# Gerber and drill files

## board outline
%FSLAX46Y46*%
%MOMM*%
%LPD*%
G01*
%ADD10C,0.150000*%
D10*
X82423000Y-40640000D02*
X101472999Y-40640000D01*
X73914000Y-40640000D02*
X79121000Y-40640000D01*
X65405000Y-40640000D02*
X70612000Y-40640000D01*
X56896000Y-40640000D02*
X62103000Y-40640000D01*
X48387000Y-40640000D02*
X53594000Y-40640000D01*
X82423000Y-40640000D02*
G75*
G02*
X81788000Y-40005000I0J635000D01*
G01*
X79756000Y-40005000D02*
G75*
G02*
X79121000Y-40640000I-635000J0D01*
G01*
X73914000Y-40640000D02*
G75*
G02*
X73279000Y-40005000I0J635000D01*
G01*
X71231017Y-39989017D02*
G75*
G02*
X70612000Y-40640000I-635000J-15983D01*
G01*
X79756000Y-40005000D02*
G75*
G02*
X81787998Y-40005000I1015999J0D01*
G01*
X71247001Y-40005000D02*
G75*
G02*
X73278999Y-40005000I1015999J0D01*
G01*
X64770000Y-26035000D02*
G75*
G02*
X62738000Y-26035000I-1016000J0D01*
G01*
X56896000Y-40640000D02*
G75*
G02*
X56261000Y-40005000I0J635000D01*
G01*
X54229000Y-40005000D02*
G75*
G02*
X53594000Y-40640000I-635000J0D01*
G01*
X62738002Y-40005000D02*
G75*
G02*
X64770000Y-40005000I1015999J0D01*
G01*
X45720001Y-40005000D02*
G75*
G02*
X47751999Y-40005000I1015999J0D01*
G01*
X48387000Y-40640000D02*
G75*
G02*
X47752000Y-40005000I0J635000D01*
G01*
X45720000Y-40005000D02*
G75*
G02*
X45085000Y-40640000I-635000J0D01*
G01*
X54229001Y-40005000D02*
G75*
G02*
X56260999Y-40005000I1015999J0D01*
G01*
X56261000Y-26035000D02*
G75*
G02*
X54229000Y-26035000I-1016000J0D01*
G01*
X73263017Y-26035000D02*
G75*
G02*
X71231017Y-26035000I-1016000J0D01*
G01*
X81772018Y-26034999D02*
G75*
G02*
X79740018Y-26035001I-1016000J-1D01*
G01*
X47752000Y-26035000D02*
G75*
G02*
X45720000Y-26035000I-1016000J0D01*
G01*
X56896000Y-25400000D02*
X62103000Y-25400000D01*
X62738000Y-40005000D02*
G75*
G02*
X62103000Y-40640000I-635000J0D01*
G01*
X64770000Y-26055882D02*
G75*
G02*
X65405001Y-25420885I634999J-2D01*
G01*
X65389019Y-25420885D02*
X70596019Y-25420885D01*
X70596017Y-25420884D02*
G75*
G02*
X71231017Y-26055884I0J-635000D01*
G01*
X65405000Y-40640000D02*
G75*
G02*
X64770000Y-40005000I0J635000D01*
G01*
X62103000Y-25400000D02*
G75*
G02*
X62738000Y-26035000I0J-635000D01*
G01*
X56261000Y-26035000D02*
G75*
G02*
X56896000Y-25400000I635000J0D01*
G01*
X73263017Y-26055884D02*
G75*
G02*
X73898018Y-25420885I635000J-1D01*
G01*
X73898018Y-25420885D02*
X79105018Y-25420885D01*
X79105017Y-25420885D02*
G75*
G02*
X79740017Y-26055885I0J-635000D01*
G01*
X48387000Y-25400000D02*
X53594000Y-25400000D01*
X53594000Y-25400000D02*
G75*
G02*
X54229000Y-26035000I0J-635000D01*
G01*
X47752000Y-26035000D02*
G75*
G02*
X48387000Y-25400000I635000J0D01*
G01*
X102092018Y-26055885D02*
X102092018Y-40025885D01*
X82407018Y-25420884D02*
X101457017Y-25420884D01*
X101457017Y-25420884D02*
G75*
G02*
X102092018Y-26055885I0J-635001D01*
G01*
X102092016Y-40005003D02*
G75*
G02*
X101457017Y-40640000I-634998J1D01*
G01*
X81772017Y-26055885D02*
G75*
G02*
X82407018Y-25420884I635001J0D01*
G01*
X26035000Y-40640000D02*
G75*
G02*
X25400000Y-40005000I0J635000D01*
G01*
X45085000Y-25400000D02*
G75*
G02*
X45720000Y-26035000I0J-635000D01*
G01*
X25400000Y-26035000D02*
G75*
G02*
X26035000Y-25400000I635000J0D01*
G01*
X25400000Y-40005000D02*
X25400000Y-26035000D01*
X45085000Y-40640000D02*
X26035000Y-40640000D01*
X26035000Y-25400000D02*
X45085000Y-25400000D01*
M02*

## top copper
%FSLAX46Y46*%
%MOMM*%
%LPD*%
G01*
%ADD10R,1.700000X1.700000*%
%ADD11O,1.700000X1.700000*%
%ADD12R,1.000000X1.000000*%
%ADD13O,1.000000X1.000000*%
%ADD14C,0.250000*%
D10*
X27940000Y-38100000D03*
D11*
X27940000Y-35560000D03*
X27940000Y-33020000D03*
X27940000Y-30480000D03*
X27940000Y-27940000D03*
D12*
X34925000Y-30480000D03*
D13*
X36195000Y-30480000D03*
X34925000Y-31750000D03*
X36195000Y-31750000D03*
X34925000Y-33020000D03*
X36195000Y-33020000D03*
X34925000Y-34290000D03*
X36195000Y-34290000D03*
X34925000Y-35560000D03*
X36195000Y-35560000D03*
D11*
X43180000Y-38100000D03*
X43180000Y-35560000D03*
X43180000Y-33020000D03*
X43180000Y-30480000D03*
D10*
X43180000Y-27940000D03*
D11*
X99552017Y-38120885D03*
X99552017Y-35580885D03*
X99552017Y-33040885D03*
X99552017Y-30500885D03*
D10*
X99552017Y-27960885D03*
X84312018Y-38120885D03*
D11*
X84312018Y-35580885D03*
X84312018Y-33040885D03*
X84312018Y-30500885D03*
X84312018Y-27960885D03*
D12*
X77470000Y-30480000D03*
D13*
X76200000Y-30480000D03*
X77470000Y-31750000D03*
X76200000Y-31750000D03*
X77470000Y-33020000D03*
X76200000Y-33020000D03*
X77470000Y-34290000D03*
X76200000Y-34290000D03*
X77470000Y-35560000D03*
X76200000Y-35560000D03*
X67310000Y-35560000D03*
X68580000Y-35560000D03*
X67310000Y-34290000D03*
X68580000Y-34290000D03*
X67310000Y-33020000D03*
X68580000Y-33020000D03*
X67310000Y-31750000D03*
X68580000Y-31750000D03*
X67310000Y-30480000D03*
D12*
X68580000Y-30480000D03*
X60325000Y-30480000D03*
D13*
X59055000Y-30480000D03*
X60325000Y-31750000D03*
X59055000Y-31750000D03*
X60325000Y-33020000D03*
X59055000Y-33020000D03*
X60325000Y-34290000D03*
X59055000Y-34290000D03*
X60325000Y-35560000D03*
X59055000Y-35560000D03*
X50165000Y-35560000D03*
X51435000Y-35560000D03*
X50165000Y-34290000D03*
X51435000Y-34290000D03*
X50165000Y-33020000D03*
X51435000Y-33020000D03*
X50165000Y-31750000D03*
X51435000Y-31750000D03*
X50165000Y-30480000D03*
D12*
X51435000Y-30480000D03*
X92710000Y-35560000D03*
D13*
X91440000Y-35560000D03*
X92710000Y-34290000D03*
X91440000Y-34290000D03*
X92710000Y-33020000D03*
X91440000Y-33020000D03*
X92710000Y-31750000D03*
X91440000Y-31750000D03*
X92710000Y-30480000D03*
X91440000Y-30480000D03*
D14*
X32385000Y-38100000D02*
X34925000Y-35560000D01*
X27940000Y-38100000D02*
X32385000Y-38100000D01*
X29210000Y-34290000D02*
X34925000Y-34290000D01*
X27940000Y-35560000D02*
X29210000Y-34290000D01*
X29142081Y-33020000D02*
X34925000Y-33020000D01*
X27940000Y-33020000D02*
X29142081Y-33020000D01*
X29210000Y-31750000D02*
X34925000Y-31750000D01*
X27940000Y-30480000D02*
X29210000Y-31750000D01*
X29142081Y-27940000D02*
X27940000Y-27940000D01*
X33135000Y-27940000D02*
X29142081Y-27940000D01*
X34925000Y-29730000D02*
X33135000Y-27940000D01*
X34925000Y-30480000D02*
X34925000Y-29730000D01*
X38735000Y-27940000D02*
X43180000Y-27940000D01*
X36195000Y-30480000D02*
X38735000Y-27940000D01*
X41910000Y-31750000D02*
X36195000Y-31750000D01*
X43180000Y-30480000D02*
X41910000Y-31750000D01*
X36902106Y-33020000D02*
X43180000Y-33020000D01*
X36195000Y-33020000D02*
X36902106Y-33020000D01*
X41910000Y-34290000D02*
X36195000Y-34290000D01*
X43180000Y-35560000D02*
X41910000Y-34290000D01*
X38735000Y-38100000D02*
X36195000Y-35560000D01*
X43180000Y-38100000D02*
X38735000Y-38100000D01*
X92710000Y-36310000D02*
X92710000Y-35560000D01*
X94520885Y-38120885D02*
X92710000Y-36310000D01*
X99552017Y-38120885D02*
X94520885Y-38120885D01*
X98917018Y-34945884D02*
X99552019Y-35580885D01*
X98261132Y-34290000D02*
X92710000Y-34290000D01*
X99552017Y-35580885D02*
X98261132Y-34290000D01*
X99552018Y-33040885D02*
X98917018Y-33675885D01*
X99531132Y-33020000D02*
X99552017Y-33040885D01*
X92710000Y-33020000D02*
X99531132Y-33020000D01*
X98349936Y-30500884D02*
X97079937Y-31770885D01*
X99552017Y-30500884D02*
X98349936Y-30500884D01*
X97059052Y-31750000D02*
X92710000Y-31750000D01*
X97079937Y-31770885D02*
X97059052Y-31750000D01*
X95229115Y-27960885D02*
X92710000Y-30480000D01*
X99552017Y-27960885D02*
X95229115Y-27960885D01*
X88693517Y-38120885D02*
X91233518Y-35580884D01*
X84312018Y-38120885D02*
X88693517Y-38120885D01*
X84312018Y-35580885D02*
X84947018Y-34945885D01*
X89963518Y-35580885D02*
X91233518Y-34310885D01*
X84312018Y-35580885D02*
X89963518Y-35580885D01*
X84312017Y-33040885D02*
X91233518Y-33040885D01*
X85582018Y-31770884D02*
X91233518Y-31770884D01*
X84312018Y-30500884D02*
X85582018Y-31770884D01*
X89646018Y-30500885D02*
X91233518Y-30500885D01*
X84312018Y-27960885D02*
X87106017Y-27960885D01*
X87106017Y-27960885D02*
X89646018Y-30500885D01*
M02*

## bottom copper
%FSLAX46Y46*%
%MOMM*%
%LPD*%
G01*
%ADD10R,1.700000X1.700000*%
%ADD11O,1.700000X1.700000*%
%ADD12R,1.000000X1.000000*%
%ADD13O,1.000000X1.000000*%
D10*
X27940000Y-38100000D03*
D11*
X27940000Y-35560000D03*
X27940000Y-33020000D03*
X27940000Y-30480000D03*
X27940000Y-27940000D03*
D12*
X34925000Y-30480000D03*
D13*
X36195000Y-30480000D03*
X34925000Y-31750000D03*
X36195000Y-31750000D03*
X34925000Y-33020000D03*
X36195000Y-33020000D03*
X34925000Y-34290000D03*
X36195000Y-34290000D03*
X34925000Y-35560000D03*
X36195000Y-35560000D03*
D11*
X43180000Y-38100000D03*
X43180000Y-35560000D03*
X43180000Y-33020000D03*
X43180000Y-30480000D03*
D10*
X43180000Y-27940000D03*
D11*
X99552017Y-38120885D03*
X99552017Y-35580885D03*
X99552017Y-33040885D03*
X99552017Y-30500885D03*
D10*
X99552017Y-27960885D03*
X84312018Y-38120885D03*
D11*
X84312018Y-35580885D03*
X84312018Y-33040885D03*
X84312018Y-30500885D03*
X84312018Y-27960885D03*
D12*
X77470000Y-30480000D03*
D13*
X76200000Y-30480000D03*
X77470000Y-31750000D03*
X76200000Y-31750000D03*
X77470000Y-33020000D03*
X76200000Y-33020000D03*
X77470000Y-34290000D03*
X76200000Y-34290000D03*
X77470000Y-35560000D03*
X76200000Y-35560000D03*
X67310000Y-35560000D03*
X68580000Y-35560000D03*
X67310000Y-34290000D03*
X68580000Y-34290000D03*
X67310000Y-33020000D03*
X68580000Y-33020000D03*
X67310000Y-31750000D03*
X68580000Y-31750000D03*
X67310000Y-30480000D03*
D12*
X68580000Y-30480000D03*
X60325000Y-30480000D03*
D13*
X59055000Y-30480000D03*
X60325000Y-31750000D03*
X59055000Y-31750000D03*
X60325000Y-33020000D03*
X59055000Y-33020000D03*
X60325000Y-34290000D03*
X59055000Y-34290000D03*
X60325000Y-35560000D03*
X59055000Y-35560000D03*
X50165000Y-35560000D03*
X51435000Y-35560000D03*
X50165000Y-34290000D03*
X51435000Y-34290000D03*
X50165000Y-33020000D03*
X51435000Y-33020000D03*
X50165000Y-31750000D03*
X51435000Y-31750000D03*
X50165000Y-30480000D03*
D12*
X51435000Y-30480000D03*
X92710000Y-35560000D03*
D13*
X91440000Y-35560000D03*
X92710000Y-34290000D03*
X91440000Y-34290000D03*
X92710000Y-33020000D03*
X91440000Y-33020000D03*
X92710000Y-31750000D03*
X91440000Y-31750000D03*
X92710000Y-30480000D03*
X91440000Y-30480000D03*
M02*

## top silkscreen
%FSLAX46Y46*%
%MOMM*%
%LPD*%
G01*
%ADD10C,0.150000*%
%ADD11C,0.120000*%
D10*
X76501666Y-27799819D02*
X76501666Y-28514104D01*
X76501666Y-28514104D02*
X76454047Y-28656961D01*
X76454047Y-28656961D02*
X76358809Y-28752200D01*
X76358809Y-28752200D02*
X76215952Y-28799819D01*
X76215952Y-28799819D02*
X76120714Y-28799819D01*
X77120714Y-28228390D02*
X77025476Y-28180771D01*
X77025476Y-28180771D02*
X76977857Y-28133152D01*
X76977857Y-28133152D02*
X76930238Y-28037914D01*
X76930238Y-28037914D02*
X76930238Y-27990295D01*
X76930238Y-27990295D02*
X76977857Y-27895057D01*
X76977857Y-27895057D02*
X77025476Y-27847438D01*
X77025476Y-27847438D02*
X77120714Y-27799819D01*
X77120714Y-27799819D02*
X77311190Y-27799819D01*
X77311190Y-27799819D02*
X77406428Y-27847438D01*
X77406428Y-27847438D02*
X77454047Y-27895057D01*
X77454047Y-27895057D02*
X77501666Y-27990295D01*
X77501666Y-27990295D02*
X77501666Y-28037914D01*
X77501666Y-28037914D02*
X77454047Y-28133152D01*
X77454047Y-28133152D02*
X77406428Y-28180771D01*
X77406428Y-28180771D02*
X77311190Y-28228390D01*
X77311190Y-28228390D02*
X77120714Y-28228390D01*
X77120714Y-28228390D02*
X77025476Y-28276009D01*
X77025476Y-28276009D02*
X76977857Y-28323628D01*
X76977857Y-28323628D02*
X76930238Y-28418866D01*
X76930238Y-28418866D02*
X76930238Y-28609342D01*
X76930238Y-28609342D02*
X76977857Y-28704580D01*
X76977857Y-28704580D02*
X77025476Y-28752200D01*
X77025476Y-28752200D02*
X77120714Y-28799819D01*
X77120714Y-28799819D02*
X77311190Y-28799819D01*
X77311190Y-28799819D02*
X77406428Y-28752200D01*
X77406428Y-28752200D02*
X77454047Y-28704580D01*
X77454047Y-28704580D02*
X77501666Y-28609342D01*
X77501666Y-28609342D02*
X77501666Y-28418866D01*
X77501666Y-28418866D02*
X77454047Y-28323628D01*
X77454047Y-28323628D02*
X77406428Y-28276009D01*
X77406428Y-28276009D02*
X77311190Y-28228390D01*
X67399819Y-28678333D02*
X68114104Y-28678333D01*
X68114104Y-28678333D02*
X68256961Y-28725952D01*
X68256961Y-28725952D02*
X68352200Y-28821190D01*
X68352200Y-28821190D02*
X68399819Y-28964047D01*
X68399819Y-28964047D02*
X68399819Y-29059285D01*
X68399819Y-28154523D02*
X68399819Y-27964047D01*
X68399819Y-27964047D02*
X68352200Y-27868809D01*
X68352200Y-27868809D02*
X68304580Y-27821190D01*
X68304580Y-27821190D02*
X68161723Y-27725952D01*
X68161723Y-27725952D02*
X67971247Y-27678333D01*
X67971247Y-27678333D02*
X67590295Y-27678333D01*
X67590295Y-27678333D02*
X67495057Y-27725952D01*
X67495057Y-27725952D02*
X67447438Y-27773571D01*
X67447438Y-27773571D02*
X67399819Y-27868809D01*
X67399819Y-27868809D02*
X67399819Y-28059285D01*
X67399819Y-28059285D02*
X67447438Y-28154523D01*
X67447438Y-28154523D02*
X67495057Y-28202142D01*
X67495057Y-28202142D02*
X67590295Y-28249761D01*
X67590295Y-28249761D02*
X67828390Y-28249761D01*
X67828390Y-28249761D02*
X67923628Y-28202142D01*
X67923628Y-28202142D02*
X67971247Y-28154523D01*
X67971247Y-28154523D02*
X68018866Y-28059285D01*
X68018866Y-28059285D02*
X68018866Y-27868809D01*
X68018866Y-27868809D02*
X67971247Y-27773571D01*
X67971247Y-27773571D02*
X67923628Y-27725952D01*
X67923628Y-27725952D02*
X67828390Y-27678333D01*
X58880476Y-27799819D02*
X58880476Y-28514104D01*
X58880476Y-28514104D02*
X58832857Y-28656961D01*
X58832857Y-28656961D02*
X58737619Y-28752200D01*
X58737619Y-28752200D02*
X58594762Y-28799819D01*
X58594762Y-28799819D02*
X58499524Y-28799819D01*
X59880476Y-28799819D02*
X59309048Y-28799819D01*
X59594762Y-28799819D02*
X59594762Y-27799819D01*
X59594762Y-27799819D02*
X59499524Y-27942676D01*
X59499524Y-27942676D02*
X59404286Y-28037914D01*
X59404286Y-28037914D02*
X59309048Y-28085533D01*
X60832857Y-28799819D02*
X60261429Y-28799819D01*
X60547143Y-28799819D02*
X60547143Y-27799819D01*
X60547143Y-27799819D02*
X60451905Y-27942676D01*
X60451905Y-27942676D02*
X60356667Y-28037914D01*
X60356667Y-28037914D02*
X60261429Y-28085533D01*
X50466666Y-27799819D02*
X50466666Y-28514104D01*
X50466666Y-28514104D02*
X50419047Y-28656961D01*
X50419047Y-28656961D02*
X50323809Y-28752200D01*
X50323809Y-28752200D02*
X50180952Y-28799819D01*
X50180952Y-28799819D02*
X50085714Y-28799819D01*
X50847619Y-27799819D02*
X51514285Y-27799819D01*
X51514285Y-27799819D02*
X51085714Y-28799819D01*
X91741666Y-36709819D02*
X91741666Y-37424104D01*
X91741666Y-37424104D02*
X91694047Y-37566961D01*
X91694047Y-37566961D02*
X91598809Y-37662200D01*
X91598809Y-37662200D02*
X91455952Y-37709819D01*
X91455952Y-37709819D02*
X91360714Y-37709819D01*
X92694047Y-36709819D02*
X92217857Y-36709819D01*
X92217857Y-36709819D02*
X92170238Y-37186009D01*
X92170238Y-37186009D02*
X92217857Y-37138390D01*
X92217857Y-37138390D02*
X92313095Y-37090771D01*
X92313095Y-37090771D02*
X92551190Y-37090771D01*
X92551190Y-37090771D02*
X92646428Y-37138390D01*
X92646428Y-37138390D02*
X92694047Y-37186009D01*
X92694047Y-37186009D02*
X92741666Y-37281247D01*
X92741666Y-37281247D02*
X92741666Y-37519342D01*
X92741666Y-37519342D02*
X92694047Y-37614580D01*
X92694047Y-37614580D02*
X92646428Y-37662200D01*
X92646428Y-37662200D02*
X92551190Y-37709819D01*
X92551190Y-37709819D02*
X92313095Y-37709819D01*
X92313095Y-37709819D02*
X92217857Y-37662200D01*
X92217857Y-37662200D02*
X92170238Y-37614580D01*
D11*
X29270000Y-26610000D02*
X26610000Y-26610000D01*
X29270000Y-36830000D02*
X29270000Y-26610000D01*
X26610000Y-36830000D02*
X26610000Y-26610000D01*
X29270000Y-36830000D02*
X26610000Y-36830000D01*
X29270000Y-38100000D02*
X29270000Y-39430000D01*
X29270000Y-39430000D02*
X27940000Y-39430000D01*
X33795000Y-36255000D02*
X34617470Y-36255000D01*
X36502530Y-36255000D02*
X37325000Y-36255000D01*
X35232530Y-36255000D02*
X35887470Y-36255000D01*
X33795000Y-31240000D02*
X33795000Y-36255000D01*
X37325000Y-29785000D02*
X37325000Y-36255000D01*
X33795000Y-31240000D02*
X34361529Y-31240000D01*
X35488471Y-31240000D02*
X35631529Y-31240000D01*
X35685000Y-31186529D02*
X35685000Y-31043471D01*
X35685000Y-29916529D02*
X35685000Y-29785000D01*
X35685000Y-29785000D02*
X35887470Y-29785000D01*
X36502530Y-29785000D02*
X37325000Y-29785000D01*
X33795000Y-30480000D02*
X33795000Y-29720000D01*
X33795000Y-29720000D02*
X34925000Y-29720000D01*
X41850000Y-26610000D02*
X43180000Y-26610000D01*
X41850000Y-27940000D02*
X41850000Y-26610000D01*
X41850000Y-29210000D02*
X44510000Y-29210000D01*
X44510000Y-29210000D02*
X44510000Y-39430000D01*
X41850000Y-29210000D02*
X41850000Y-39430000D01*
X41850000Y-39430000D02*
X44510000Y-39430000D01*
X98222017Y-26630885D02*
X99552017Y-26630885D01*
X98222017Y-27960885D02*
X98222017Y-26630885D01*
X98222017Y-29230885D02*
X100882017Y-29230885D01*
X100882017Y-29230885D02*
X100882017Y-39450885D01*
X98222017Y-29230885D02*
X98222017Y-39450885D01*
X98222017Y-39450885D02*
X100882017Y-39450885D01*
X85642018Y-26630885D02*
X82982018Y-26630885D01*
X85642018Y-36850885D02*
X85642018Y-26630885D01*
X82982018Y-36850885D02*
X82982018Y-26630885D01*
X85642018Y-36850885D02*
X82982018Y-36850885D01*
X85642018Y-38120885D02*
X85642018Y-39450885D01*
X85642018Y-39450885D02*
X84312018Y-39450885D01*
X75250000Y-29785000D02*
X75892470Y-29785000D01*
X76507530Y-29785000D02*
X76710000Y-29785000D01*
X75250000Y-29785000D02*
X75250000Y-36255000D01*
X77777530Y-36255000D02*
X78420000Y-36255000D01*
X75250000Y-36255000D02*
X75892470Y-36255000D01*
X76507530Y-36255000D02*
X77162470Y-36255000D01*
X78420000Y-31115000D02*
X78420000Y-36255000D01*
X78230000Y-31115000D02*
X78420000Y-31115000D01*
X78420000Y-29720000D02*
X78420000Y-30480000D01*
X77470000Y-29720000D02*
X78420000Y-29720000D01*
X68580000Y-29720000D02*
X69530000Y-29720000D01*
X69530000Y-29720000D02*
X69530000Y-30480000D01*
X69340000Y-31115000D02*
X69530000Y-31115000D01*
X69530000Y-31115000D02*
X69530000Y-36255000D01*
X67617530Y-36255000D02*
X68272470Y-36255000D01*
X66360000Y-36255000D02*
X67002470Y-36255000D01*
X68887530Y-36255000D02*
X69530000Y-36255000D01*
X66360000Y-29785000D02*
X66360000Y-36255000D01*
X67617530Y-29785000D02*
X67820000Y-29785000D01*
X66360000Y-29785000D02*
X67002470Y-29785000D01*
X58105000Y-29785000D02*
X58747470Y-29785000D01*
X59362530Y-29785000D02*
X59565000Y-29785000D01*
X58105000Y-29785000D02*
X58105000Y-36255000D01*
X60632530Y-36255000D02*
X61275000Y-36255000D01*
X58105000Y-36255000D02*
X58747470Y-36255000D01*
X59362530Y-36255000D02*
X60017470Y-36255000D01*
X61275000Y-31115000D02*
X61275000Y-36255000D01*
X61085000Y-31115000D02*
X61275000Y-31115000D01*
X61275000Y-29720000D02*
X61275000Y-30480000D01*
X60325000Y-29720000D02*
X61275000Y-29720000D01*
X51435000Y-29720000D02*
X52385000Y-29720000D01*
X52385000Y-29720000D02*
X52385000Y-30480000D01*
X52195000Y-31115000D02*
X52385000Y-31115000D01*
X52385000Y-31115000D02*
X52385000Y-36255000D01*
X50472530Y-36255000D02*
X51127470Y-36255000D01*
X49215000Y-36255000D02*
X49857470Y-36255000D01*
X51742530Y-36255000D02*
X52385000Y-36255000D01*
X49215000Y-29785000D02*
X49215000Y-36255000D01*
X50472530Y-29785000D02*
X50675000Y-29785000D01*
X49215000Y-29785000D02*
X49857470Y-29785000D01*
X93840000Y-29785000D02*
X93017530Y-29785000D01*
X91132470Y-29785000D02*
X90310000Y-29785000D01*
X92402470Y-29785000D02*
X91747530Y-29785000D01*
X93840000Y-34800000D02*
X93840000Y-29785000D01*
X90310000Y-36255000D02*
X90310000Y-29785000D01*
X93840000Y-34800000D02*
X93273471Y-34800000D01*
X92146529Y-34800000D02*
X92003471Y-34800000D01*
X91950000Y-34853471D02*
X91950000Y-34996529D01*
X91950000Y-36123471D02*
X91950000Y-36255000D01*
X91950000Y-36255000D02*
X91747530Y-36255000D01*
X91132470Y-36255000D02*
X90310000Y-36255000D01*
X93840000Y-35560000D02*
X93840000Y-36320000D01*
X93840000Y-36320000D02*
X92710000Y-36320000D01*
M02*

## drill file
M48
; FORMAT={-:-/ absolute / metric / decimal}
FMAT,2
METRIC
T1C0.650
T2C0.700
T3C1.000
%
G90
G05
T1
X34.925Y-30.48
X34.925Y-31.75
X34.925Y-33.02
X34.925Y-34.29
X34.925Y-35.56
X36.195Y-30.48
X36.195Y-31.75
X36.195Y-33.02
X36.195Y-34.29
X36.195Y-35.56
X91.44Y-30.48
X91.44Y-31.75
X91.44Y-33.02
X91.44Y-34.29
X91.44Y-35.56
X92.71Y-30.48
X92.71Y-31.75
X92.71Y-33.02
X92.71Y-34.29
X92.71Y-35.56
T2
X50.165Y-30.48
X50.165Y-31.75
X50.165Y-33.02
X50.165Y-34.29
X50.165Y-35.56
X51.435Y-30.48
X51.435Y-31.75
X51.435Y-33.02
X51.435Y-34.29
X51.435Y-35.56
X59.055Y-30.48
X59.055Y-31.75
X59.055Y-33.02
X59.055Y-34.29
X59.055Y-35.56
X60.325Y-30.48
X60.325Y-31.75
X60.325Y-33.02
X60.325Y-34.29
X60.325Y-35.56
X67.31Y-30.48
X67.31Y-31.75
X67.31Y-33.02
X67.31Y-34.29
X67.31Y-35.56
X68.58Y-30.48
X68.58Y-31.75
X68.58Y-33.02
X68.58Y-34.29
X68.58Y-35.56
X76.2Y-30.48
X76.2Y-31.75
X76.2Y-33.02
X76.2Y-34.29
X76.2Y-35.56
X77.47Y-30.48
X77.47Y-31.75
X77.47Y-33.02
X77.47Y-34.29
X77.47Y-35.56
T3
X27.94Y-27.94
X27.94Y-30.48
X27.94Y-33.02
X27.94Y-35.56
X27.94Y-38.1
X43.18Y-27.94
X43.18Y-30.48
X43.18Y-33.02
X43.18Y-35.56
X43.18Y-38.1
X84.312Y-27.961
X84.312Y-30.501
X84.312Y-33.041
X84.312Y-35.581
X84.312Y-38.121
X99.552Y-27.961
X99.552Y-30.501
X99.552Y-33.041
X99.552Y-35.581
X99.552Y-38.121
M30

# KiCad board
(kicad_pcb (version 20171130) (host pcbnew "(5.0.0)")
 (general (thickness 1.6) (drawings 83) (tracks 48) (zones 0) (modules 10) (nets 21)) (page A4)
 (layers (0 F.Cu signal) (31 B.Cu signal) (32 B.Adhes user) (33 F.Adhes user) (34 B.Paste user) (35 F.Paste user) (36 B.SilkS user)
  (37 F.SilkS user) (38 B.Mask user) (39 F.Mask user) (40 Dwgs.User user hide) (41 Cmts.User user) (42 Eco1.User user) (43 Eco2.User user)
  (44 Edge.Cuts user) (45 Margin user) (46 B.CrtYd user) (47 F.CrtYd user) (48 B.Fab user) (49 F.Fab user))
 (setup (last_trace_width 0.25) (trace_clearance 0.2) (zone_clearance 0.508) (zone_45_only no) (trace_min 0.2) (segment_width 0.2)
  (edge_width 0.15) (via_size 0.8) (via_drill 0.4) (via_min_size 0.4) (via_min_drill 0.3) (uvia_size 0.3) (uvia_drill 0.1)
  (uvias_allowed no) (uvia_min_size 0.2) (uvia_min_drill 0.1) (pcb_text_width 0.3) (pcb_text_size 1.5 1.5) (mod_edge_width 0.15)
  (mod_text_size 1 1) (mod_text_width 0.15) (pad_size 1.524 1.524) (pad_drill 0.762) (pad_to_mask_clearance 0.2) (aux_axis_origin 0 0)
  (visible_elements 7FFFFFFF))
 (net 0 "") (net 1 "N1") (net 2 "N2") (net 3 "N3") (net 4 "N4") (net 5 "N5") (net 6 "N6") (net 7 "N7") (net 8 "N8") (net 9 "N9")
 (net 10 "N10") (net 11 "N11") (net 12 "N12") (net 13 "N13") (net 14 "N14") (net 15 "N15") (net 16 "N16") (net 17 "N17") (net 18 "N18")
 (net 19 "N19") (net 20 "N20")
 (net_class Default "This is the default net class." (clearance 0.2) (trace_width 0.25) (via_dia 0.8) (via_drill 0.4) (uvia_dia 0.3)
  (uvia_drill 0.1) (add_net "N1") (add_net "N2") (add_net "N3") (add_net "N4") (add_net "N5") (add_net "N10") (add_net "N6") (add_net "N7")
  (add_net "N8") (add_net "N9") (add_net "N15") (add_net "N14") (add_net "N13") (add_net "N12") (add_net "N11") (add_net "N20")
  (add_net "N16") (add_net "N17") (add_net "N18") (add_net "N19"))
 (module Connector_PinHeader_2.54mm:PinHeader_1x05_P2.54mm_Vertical (layer F.Cu) (at 27.94 38.1 180)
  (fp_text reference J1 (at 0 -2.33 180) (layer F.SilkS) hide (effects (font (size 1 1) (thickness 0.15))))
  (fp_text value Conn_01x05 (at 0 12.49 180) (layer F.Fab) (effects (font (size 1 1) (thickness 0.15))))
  (fp_line (start -1.33 11.49) (end 1.33 11.49) (layer F.SilkS) (width 0.12))
  (fp_line (start -1.33 1.27) (end -1.33 11.49) (layer F.SilkS) (width 0.12))
  (fp_line (start 1.33 1.27) (end 1.33 11.49) (layer F.SilkS) (width 0.12))
  (fp_line (start -1.33 1.27) (end 1.33 1.27) (layer F.SilkS) (width 0.12))
  (fp_line (start -1.33 0) (end -1.33 -1.33) (layer F.SilkS) (width 0.12))
  (fp_line (start -1.33 -1.33) (end 0 -1.33) (layer F.SilkS) (width 0.12))
  (pad 1 thru_hole rect (at 0 0 180) (size 1.7 1.7) (drill 1) (layers *.Cu *.Mask) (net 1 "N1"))
  (pad 2 thru_hole oval (at 0 2.54 180) (size 1.7 1.7) (drill 1) (layers *.Cu *.Mask) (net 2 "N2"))
  (pad 3 thru_hole oval (at 0 5.08 180) (size 1.7 1.7) (drill 1) (layers *.Cu *.Mask) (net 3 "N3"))
  (pad 4 thru_hole oval (at 0 7.62 180) (size 1.7 1.7) (drill 1) (layers *.Cu *.Mask) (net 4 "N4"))
  (pad 5 thru_hole oval (at 0 10.16 180) (size 1.7 1.7) (drill 1) (layers *.Cu *.Mask) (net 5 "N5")))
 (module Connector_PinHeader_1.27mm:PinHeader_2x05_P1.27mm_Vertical (layer F.Cu) (at 34.925 30.48)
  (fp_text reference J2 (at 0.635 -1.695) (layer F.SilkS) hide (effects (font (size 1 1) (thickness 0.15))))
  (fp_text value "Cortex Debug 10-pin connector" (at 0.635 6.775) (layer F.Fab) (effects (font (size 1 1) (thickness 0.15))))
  (fp_line (start -1.13 5.775) (end -0.30753 5.775) (layer F.SilkS) (width 0.12))
  (fp_line (start 1.57753 5.775) (end 2.4 5.775) (layer F.SilkS) (width 0.12))
  (fp_line (start 0.30753 5.775) (end 0.96247 5.775) (layer F.SilkS) (width 0.12))
  (fp_line (start -1.13 0.76) (end -1.13 5.775) (layer F.SilkS) (width 0.12))
  (fp_line (start 2.4 -0.695) (end 2.4 5.775) (layer F.SilkS) (width 0.12))
  (fp_line (start -1.13 0.76) (end -0.563471 0.76) (layer F.SilkS) (width 0.12))
  (fp_line (start 0.563471 0.76) (end 0.706529 0.76) (layer F.SilkS) (width 0.12))
  (fp_line (start 0.76 0.706529) (end 0.76 0.563471) (layer F.SilkS) (width 0.12))
  (fp_line (start 0.76 -0.563471) (end 0.76 -0.695) (layer F.SilkS) (width 0.12))
  (fp_line (start 0.76 -0.695) (end 0.96247 -0.695) (layer F.SilkS) (width 0.12))
  (fp_line (start 1.57753 -0.695) (end 2.4 -0.695) (layer F.SilkS) (width 0.12))
  (fp_line (start -1.13 0) (end -1.13 -0.76) (layer F.SilkS) (width 0.12))
  (fp_line (start -1.13 -0.76) (end 0 -0.76) (layer F.SilkS) (width 0.12))
  (pad 1 thru_hole rect (at 0 0) (size 1 1) (drill 0.65) (layers *.Cu *.Mask) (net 5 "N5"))
  (pad 2 thru_hole oval (at 1.27 0) (size 1 1) (drill 0.65) (layers *.Cu *.Mask) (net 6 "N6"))
  (pad 3 thru_hole oval (at 0 1.27) (size 1 1) (drill 0.65) (layers *.Cu *.Mask) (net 4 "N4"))
  (pad 4 thru_hole oval (at 1.27 1.27) (size 1 1) (drill 0.65) (layers *.Cu *.Mask) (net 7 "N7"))
  (pad 5 thru_hole oval (at 0 2.54) (size 1 1) (drill 0.65) (layers *.Cu *.Mask) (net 3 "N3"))
  (pad 6 thru_hole oval (at 1.27 2.54) (size 1 1) (drill 0.65) (layers *.Cu *.Mask) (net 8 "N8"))
  (pad 7 thru_hole oval (at 0 3.81) (size 1 1) (drill 0.65) (layers *.Cu *.Mask) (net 2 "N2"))
  (pad 8 thru_hole oval (at 1.27 3.81) (size 1 1) (drill 0.65) (layers *.Cu *.Mask) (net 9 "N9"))
  (pad 9 thru_hole oval (at 0 5.08) (size 1 1) (drill 0.65) (layers *.Cu *.Mask) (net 1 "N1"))
  (pad 10 thru_hole oval (at 1.27 5.08) (size 1 1) (drill 0.65) (layers *.Cu *.Mask) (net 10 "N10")))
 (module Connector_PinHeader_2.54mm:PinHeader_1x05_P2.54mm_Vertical (layer F.Cu) (at 43.18 27.94)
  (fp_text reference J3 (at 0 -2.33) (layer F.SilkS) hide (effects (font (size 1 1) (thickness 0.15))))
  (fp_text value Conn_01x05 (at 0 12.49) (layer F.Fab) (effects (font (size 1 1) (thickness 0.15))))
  (fp_line (start -1.33 -1.33) (end 0 -1.33) (layer F.SilkS) (width 0.12))
  (fp_line (start -1.33 0) (end -1.33 -1.33) (layer F.SilkS) (width 0.12))
  (fp_line (start -1.33 1.27) (end 1.33 1.27) (layer F.SilkS) (width 0.12))
  (fp_line (start 1.33 1.27) (end 1.33 11.49) (layer F.SilkS) (width 0.12))
  (fp_line (start -1.33 1.27) (end -1.33 11.49) (layer F.SilkS) (width 0.12))
  (fp_line (start -1.33 11.49) (end 1.33 11.49) (layer F.SilkS) (width 0.12))
  (pad 5 thru_hole oval (at 0 10.16) (size 1.7 1.7) (drill 1) (layers *.Cu *.Mask) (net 10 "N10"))
  (pad 4 thru_hole oval (at 0 7.62) (size 1.7 1.7) (drill 1) (layers *.Cu *.Mask) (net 9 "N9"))
  (pad 3 thru_hole oval (at 0 5.08) (size 1.7 1.7) (drill 1) (layers *.Cu *.Mask) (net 8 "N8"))
  (pad 2 thru_hole oval (at 0 2.54) (size 1.7 1.7) (drill 1) (layers *.Cu *.Mask) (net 7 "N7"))
  (pad 1 thru_hole rect (at 0 0) (size 1.7 1.7) (drill 1) (layers *.Cu *.Mask) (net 6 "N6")))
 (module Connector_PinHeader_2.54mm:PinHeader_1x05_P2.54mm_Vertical (layer F.Cu) (at 99.552017 27.960885)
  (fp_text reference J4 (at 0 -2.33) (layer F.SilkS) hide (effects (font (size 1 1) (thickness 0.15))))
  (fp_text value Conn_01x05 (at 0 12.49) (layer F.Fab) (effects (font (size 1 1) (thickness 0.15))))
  (fp_line (start -1.33 -1.33) (end 0 -1.33) (layer F.SilkS) (width 0.12))
  (fp_line (start -1.33 0) (end -1.33 -1.33) (layer F.SilkS) (width 0.12))
  (fp_line (start -1.33 1.27) (end 1.33 1.27) (layer F.SilkS) (width 0.12))
  (fp_line (start 1.33 1.27) (end 1.33 11.49) (layer F.SilkS) (width 0.12))
  (fp_line (start -1.33 1.27) (end -1.33 11.49) (layer F.SilkS) (width 0.12))
  (fp_line (start -1.33 11.49) (end 1.33 11.49) (layer F.SilkS) (width 0.12))
  (pad 5 thru_hole oval (at 0 10.16) (size 1.7 1.7) (drill 1) (layers *.Cu *.Mask) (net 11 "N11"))
  (pad 4 thru_hole oval (at 0 7.62) (size 1.7 1.7) (drill 1) (layers *.Cu *.Mask) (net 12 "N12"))
  (pad 3 thru_hole oval (at 0 5.08) (size 1.7 1.7) (drill 1) (layers *.Cu *.Mask) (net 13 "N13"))
  (pad 2 thru_hole oval (at 0 2.54) (size 1.7 1.7) (drill 1) (layers *.Cu *.Mask) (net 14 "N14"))
  (pad 1 thru_hole rect (at 0 0) (size 1.7 1.7) (drill 1) (layers *.Cu *.Mask) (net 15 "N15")))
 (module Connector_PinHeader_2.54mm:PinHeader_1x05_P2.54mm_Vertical (layer F.Cu) (at 84.312018 38.120885 180)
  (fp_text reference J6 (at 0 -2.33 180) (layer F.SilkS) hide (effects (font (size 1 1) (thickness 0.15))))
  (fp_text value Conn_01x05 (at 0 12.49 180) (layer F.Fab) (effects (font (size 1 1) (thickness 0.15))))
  (fp_line (start -1.33 11.49) (end 1.33 11.49) (layer F.SilkS) (width 0.12))
  (fp_line (start -1.33 1.27) (end -1.33 11.49) (layer F.SilkS) (width 0.12))
  (fp_line (start 1.33 1.27) (end 1.33 11.49) (layer F.SilkS) (width 0.12))
  (fp_line (start -1.33 1.27) (end 1.33 1.27) (layer F.SilkS) (width 0.12))
  (fp_line (start -1.33 0) (end -1.33 -1.33) (layer F.SilkS) (width 0.12))
  (fp_line (start -1.33 -1.33) (end 0 -1.33) (layer F.SilkS) (width 0.12))
  (pad 1 thru_hole rect (at 0 0 180) (size 1.7 1.7) (drill 1) (layers *.Cu *.Mask) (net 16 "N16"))
  (pad 2 thru_hole oval (at 0 2.54 180) (size 1.7 1.7) (drill 1) (layers *.Cu *.Mask) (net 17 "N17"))
  (pad 3 thru_hole oval (at 0 5.08 180) (size 1.7 1.7) (drill 1) (layers *.Cu *.Mask) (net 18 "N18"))
  (pad 4 thru_hole oval (at 0 7.62 180) (size 1.7 1.7) (drill 1) (layers *.Cu *.Mask) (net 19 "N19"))
  (pad 5 thru_hole oval (at 0 10.16 180) (size 1.7 1.7) (drill 1) (layers *.Cu *.Mask) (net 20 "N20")))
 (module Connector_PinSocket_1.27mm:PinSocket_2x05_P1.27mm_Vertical (layer F.Cu) (at 77.47 30.48)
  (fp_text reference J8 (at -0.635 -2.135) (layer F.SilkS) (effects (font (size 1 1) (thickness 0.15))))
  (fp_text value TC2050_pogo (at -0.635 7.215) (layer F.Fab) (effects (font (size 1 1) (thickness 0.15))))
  (fp_line (start -2.22 -0.695) (end -1.57753 -0.695) (layer F.SilkS) (width 0.12))
  (fp_line (start -0.96247 -0.695) (end -0.76 -0.695) (layer F.SilkS) (width 0.12))
  (fp_line (start -2.22 -0.695) (end -2.22 5.775) (layer F.SilkS) (width 0.12))
  (fp_line (start 0.30753 5.775) (end 0.95 5.775) (layer F.SilkS) (width 0.12))
  (fp_line (start -2.22 5.775) (end -1.57753 5.775) (layer F.SilkS) (width 0.12))
  (fp_line (start -0.96247 5.775) (end -0.30753 5.775) (layer F.SilkS) (width 0.12))
  (fp_line (start 0.95 0.635) (end 0.95 5.775) (layer F.SilkS) (width 0.12))
  (fp_line (start 0.76 0.635) (end 0.95 0.635) (layer F.SilkS) (width 0.12))
  (fp_line (start 0.95 -0.76) (end 0.95 0) (layer F.SilkS) (width 0.12))
  (fp_line (start 0 -0.76) (end 0.95 -0.76) (layer F.SilkS) (width 0.12))
  (pad 1 thru_hole rect (at 0 0) (size 1 1) (drill 0.7) (layers *.Cu *.Mask))
  (pad 2 thru_hole oval (at -1.27 0) (size 1 1) (drill 0.7) (layers *.Cu *.Mask))
  (pad 3 thru_hole oval (at 0 1.27) (size 1 1) (drill 0.7) (layers *.Cu *.Mask))
  (pad 4 thru_hole oval (at -1.27 1.27) (size 1 1) (drill 0.7) (layers *.Cu *.Mask))
  (pad 5 thru_hole oval (at 0 2.54) (size 1 1) (drill 0.7) (layers *.Cu *.Mask))
  (pad 6 thru_hole oval (at -1.27 2.54) (size 1 1) (drill 0.7) (layers *.Cu *.Mask))
  (pad 7 thru_hole oval (at 0 3.81) (size 1 1) (drill 0.7) (layers *.Cu *.Mask))
  (pad 8 thru_hole oval (at -1.27 3.81) (size 1 1) (drill 0.7) (layers *.Cu *.Mask))
  (pad 9 thru_hole oval (at 0 5.08) (size 1 1) (drill 0.7) (layers *.Cu *.Mask))
  (pad 10 thru_hole oval (at -1.27 5.08) (size 1 1) (drill 0.7) (layers *.Cu *.Mask)))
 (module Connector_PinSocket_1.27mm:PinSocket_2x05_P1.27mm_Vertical (layer F.Cu) (at 68.58 30.48)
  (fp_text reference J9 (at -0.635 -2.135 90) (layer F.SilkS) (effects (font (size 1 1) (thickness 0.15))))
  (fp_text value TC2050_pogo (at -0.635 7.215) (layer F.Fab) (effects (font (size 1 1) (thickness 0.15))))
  (fp_line (start 0 -0.76) (end 0.95 -0.76) (layer F.SilkS) (width 0.12))
  (fp_line (start 0.95 -0.76) (end 0.95 0) (layer F.SilkS) (width 0.12))
  (fp_line (start 0.76 0.635) (end 0.95 0.635) (layer F.SilkS) (width 0.12))
  (fp_line (start 0.95 0.635) (end 0.95 5.775) (layer F.SilkS) (width 0.12))
  (fp_line (start -0.96247 5.775) (end -0.30753 5.775) (layer F.SilkS) (width 0.12))
  (fp_line (start -2.22 5.775) (end -1.57753 5.775) (layer F.SilkS) (width 0.12))
  (fp_line (start 0.30753 5.775) (end 0.95 5.775) (layer F.SilkS) (width 0.12))
  (fp_line (start -2.22 -0.695) (end -2.22 5.775) (layer F.SilkS) (width 0.12))
  (fp_line (start -0.96247 -0.695) (end -0.76 -0.695) (layer F.SilkS) (width 0.12))
  (fp_line (start -2.22 -0.695) (end -1.57753 -0.695) (layer F.SilkS) (width 0.12))
  (pad 10 thru_hole oval (at -1.27 5.08) (size 1 1) (drill 0.7) (layers *.Cu *.Mask))
  (pad 9 thru_hole oval (at 0 5.08) (size 1 1) (drill 0.7) (layers *.Cu *.Mask))
  (pad 8 thru_hole oval (at -1.27 3.81) (size 1 1) (drill 0.7) (layers *.Cu *.Mask))
  (pad 7 thru_hole oval (at 0 3.81) (size 1 1) (drill 0.7) (layers *.Cu *.Mask))
  (pad 6 thru_hole oval (at -1.27 2.54) (size 1 1) (drill 0.7) (layers *.Cu *.Mask))
  (pad 5 thru_hole oval (at 0 2.54) (size 1 1) (drill 0.7) (layers *.Cu *.Mask))
  (pad 4 thru_hole oval (at -1.27 1.27) (size 1 1) (drill 0.7) (layers *.Cu *.Mask))
  (pad 3 thru_hole oval (at 0 1.27) (size 1 1) (drill 0.7) (layers *.Cu *.Mask))
  (pad 2 thru_hole oval (at -1.27 0) (size 1 1) (drill 0.7) (layers *.Cu *.Mask))
  (pad 1 thru_hole rect (at 0 0) (size 1 1) (drill 0.7) (layers *.Cu *.Mask)))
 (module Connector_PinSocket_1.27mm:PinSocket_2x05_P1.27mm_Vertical (layer F.Cu) (at 60.325 30.48)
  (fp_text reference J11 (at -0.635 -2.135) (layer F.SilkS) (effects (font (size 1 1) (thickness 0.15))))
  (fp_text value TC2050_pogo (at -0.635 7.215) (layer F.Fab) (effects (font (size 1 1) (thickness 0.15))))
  (fp_line (start -2.22 -0.695) (end -1.57753 -0.695) (layer F.SilkS) (width 0.12))
  (fp_line (start -0.96247 -0.695) (end -0.76 -0.695) (layer F.SilkS) (width 0.12))
  (fp_line (start -2.22 -0.695) (end -2.22 5.775) (layer F.SilkS) (width 0.12))
  (fp_line (start 0.30753 5.775) (end 0.95 5.775) (layer F.SilkS) (width 0.12))
  (fp_line (start -2.22 5.775) (end -1.57753 5.775) (layer F.SilkS) (width 0.12))
  (fp_line (start -0.96247 5.775) (end -0.30753 5.775) (layer F.SilkS) (width 0.12))
  (fp_line (start 0.95 0.635) (end 0.95 5.775) (layer F.SilkS) (width 0.12))
  (fp_line (start 0.76 0.635) (end 0.95 0.635) (layer F.SilkS) (width 0.12))
  (fp_line (start 0.95 -0.76) (end 0.95 0) (layer F.SilkS) (width 0.12))
  (fp_line (start 0 -0.76) (end 0.95 -0.76) (layer F.SilkS) (width 0.12))
  (pad 1 thru_hole rect (at 0 0) (size 1 1) (drill 0.7) (layers *.Cu *.Mask))
  (pad 2 thru_hole oval (at -1.27 0) (size 1 1) (drill 0.7) (layers *.Cu *.Mask))
  (pad 3 thru_hole oval (at 0 1.27) (size 1 1) (drill 0.7) (layers *.Cu *.Mask))
  (pad 4 thru_hole oval (at -1.27 1.27) (size 1 1) (drill 0.7) (layers *.Cu *.Mask))
  (pad 5 thru_hole oval (at 0 2.54) (size 1 1) (drill 0.7) (layers *.Cu *.Mask))
  (pad 6 thru_hole oval (at -1.27 2.54) (size 1 1) (drill 0.7) (layers *.Cu *.Mask))
  (pad 7 thru_hole oval (at 0 3.81) (size 1 1) (drill 0.7) (layers *.Cu *.Mask))
  (pad 8 thru_hole oval (at -1.27 3.81) (size 1 1) (drill 0.7) (layers *.Cu *.Mask))
  (pad 9 thru_hole oval (at 0 5.08) (size 1 1) (drill 0.7) (layers *.Cu *.Mask))
  (pad 10 thru_hole oval (at -1.27 5.08) (size 1 1) (drill 0.7) (layers *.Cu *.Mask)))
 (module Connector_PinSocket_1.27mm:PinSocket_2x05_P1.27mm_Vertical (layer F.Cu) (at 51.435 30.48)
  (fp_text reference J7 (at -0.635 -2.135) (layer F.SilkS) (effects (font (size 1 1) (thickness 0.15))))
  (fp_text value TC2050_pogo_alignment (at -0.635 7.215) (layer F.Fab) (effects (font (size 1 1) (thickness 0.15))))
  (fp_line (start 0 -0.76) (end 0.95 -0.76) (layer F.SilkS) (width 0.12))
  (fp_line (start 0.95 -0.76) (end 0.95 0) (layer F.SilkS) (width 0.12))
  (fp_line (start 0.76 0.635) (end 0.95 0.635) (layer F.SilkS) (width 0.12))
  (fp_line (start 0.95 0.635) (end 0.95 5.775) (layer F.SilkS) (width 0.12))
  (fp_line (start -0.96247 5.775) (end -0.30753 5.775) (layer F.SilkS) (width 0.12))
  (fp_line (start -2.22 5.775) (end -1.57753 5.775) (layer F.SilkS) (width 0.12))
  (fp_line (start 0.30753 5.775) (end 0.95 5.775) (layer F.SilkS) (width 0.12))
  (fp_line (start -2.22 -0.695) (end -2.22 5.775) (layer F.SilkS) (width 0.12))
  (fp_line (start -0.96247 -0.695) (end -0.76 -0.695) (layer F.SilkS) (width 0.12))
  (fp_line (start -2.22 -0.695) (end -1.57753 -0.695) (layer F.SilkS) (width 0.12))
  (pad 10 thru_hole oval (at -1.27 5.08) (size 1 1) (drill 0.7) (layers *.Cu *.Mask))
  (pad 9 thru_hole oval (at 0 5.08) (size 1 1) (drill 0.7) (layers *.Cu *.Mask))
  (pad 8 thru_hole oval (at -1.27 3.81) (size 1 1) (drill 0.7) (layers *.Cu *.Mask))
  (pad 7 thru_hole oval (at 0 3.81) (size 1 1) (drill 0.7) (layers *.Cu *.Mask))
  (pad 6 thru_hole oval (at -1.27 2.54) (size 1 1) (drill 0.7) (layers *.Cu *.Mask))
  (pad 5 thru_hole oval (at 0 2.54) (size 1 1) (drill 0.7) (layers *.Cu *.Mask))
  (pad 4 thru_hole oval (at -1.27 1.27) (size 1 1) (drill 0.7) (layers *.Cu *.Mask))
  (pad 3 thru_hole oval (at 0 1.27) (size 1 1) (drill 0.7) (layers *.Cu *.Mask))
  (pad 2 thru_hole oval (at -1.27 0) (size 1 1) (drill 0.7) (layers *.Cu *.Mask))
  (pad 1 thru_hole rect (at 0 0) (size 1 1) (drill 0.7) (layers *.Cu *.Mask)))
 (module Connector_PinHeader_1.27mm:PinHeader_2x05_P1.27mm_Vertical (layer F.Cu) (at 92.71 35.56 180)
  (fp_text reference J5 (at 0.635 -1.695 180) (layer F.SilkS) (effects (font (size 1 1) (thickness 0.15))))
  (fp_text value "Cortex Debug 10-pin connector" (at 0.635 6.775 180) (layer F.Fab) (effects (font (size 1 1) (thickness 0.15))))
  (fp_line (start -1.13 5.775) (end -0.30753 5.775) (layer F.SilkS) (width 0.12))
  (fp_line (start 1.57753 5.775) (end 2.4 5.775) (layer F.SilkS) (width 0.12))
  (fp_line (start 0.30753 5.775) (end 0.96247 5.775) (layer F.SilkS) (width 0.12))
  (fp_line (start -1.13 0.76) (end -1.13 5.775) (layer F.SilkS) (width 0.12))
  (fp_line (start 2.4 -0.695) (end 2.4 5.775) (layer F.SilkS) (width 0.12))
  (fp_line (start -1.13 0.76) (end -0.563471 0.76) (layer F.SilkS) (width 0.12))
  (fp_line (start 0.563471 0.76) (end 0.706529 0.76) (layer F.SilkS) (width 0.12))
  (fp_line (start 0.76 0.706529) (end 0.76 0.563471) (layer F.SilkS) (width 0.12))
  (fp_line (start 0.76 -0.563471) (end 0.76 -0.695) (layer F.SilkS) (width 0.12))
  (fp_line (start 0.76 -0.695) (end 0.96247 -0.695) (layer F.SilkS) (width 0.12))
  (fp_line (start 1.57753 -0.695) (end 2.4 -0.695) (layer F.SilkS) (width 0.12))
  (fp_line (start -1.13 0) (end -1.13 -0.76) (layer F.SilkS) (width 0.12))
  (fp_line (start -1.13 -0.76) (end 0 -0.76) (layer F.SilkS) (width 0.12))
  (pad 1 thru_hole rect (at 0 0 180) (size 1 1) (drill 0.65) (layers *.Cu *.Mask) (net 11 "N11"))
  (pad 2 thru_hole oval (at 1.27 0 180) (size 1 1) (drill 0.65) (layers *.Cu *.Mask) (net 16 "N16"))
  (pad 3 thru_hole oval (at 0 1.27 180) (size 1 1) (drill 0.65) (layers *.Cu *.Mask) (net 12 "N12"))
  (pad 4 thru_hole oval (at 1.27 1.27 180) (size 1 1) (drill 0.65) (layers *.Cu *.Mask) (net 17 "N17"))
  (pad 5 thru_hole oval (at 0 2.54 180) (size 1 1) (drill 0.65) (layers *.Cu *.Mask) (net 13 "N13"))
  (pad 6 thru_hole oval (at 1.27 2.54 180) (size 1 1) (drill 0.65) (layers *.Cu *.Mask) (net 18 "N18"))
  (pad 7 thru_hole oval (at 0 3.81 180) (size 1 1) (drill 0.65) (layers *.Cu *.Mask) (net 14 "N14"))
  (pad 8 thru_hole oval (at 1.27 3.81 180) (size 1 1) (drill 0.65) (layers *.Cu *.Mask) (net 19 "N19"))
  (pad 9 thru_hole oval (at 0 5.08 180) (size 1 1) (drill 0.65) (layers *.Cu *.Mask) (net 15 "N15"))
  (pad 10 thru_hole oval (at 1.27 5.08 180) (size 1 1) (drill 0.65) (layers *.Cu *.Mask) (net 20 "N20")))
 (gr_line (start 82.423 40.64) (end 101.472999 40.64) (layer Edge.Cuts) (width 0.15))
 (gr_line (start 73.914 40.64) (end 79.121 40.64) (layer Edge.Cuts) (width 0.15))
 (gr_line (start 65.405 40.64) (end 70.612 40.64) (layer Edge.Cuts) (width 0.15))
 (gr_line (start 56.896 40.64) (end 62.103 40.64) (layer Edge.Cuts) (width 0.15))
 (gr_line (start 48.387 40.64) (end 53.594 40.64) (layer Edge.Cuts) (width 0.15))
 (gr_arc (start 82.423 40.005) (end 81.788 40.005) (angle -90) (layer Edge.Cuts) (width 0.15))
 (gr_arc (start 79.121 40.005) (end 79.121 40.64) (angle -90) (layer Edge.Cuts) (width 0.15))
 (gr_arc (start 73.914 40.005) (end 73.279 40.005) (angle -90) (layer Edge.Cuts) (width 0.15))
 (gr_arc (start 70.596017 40.005) (end 70.612 40.64) (angle -90) (layer Edge.Cuts) (width 0.15))
 (gr_arc (start 80.771999 40.005) (end 81.787998 40.005) (angle -180) (layer Edge.Cuts) (width 0.15))
 (gr_arc (start 72.263 40.005) (end 73.278999 40.005) (angle -180) (layer Edge.Cuts) (width 0.15))
 (gr_arc (start 63.754 26.035) (end 62.738 26.035) (angle -180) (layer Edge.Cuts) (width 0.15))
 (gr_arc (start 56.896 40.005) (end 56.261 40.005) (angle -90) (layer Edge.Cuts) (width 0.15))
 (gr_arc (start 53.594 40.005) (end 53.594 40.64) (angle -90) (layer Edge.Cuts) (width 0.15))
 (gr_arc (start 63.754001 40.005) (end 64.77 40.005) (angle -180) (layer Edge.Cuts) (width 0.15))
 (gr_arc (start 46.736 40.005) (end 47.751999 40.005) (angle -180) (layer Edge.Cuts) (width 0.15))
 (gr_arc (start 48.387 40.005) (end 47.752 40.005) (angle -90) (layer Edge.Cuts) (width 0.15))
 (gr_arc (start 45.085 40.005) (end 45.085 40.64) (angle -90) (layer Edge.Cuts) (width 0.15))
 (gr_arc (start 55.245 40.005) (end 56.260999 40.005) (angle -180) (layer Edge.Cuts) (width 0.15))
 (gr_arc (start 55.245 26.035) (end 54.229 26.035) (angle -180) (layer Edge.Cuts) (width 0.15))
 (gr_arc (start 72.247017 26.035) (end 71.231017 26.035) (angle -180) (layer Edge.Cuts) (width 0.15))
 (gr_arc (start 80.756018 26.035) (end 79.740018 26.035001) (angle -180) (layer Edge.Cuts) (width 0.15))
 (gr_arc (start 46.736 26.035) (end 45.72 26.035) (angle -180) (layer Edge.Cuts) (width 0.15))
 (gr_line (start 56.896 25.4) (end 62.103 25.4) (layer Edge.Cuts) (width 0.15))
 (gr_arc (start 62.103 40.005) (end 62.103 40.64) (angle -90) (layer Edge.Cuts) (width 0.15))
 (gr_arc (start 65.404999 26.055884) (end 65.405001 25.420885) (angle -90) (layer Edge.Cuts) (width 0.15))
 (gr_line (start 65.389019 25.420885) (end 70.596019 25.420885) (layer Edge.Cuts) (width 0.15))
 (gr_arc (start 70.596017 26.055884) (end 71.231017 26.055884) (angle -90) (layer Edge.Cuts) (width 0.15))
 (gr_arc (start 65.405 40.005) (end 64.77 40.005) (angle -90) (layer Edge.Cuts) (width 0.15))
 (gr_arc (start 62.103 26.035) (end 62.738 26.035) (angle -90) (layer Edge.Cuts) (width 0.15))
 (gr_arc (start 56.896 26.035) (end 56.896 25.4) (angle -90) (layer Edge.Cuts) (width 0.15))
 (gr_arc (start 73.898017 26.055885) (end 73.898018 25.420885) (angle -90) (layer Edge.Cuts) (width 0.15))
 (gr_line (start 73.898018 25.420885) (end 79.105018 25.420885) (layer Edge.Cuts) (width 0.15))
 (gr_arc (start 79.105017 26.055885) (end 79.740017 26.055885) (angle -90) (layer Edge.Cuts) (width 0.15))
 (gr_line (start 48.387 25.4) (end 53.594 25.4) (layer Edge.Cuts) (width 0.15))
 (gr_arc (start 53.594 26.035) (end 54.229 26.035) (angle -90) (layer Edge.Cuts) (width 0.15))
 (gr_arc (start 48.387 26.035) (end 48.387 25.4) (angle -90) (layer Edge.Cuts) (width 0.15))
 (gr_line (start 102.092018 26.055885) (end 102.092018 40.025885) (layer Edge.Cuts) (width 0.15))
 (gr_line (start 82.407018 25.420884) (end 101.457017 25.420884) (layer Edge.Cuts) (width 0.15))
 (gr_arc (start 101.457017 26.055885) (end 102.092018 26.055885) (angle -90) (layer Edge.Cuts) (width 0.15))
 (gr_arc (start 101.457018 40.005002) (end 101.457017 40.64) (angle -90) (layer Edge.Cuts) (width 0.15))
 (gr_arc (start 82.407018 26.055885) (end 82.407018 25.420884) (angle -90) (layer Edge.Cuts) (width 0.15))
 (gr_arc (start 26.035 40.005) (end 25.4 40.005) (angle -90) (layer Edge.Cuts) (width 0.15))
 (gr_arc (start 45.085 26.035) (end 45.72 26.035) (angle -90) (layer Edge.Cuts) (width 0.15))
 (gr_arc (start 26.035 26.035) (end 26.035 25.4) (angle -90) (layer Edge.Cuts) (width 0.15))
 (gr_line (start 25.4 40.005) (end 25.4 26.035) (layer Edge.Cuts) (width 0.15))
 (gr_line (start 45.085 40.64) (end 26.035 40.64) (layer Edge.Cuts) (width 0.15))
 (gr_line (start 26.035 25.4) (end 45.085 25.4) (layer Edge.Cuts) (width 0.15))
 (segment (start 32.385 38.1) (end 34.925 35.56) (width 0.25) (layer F.Cu) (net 1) (status 20))
 (segment (start 27.94 38.1) (end 32.385 38.1) (width 0.25) (layer F.Cu) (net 1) (status 10))
 (segment (start 29.21 34.29) (end 34.925 34.29) (width 0.25) (layer F.Cu) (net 2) (status 20))
 (segment (start 27.94 35.56) (end 29.21 34.29) (width 0.25) (layer F.Cu) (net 2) (status 10))
 (segment (start 29.142081 33.02) (end 34.925 33.02) (width 0.25) (layer F.Cu) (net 3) (status 20))
 (segment (start 27.94 33.02) (end 29.142081 33.02) (width 0.25) (layer F.Cu) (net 3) (status 10))
 (segment (start 29.21 31.75) (end 34.925 31.75) (width 0.25) (layer F.Cu) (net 4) (status 20))
 (segment (start 27.94 30.48) (end 29.21 31.75) (width 0.25) (layer F.Cu) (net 4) (status 10))
 (segment (start 29.142081 27.94) (end 27.94 27.94) (width 0.25) (layer F.Cu) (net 5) (status 20))
 (segment (start 33.135 27.94) (end 29.142081 27.94) (width 0.25) (layer F.Cu) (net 5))
 (segment (start 34.925 29.73) (end 33.135 27.94) (width 0.25) (layer F.Cu) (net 5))
 (segment (start 34.925 30.48) (end 34.925 29.73) (width 0.25) (layer F.Cu) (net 5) (status 10))
 (segment (start 38.735 27.94) (end 43.18 27.94) (width 0.25) (layer F.Cu) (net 6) (status 20))
 (segment (start 36.195 30.48) (end 38.735 27.94) (width 0.25) (layer F.Cu) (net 6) (status 10))
 (segment (start 41.91 31.75) (end 36.195 31.75) (width 0.25) (layer F.Cu) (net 7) (status 20))
 (segment (start 43.18 30.48) (end 41.91 31.75) (width 0.25) (layer F.Cu) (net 7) (status 10))
 (segment (start 36.902106 33.02) (end 43.18 33.02) (width 0.25) (layer F.Cu) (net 8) (status 20))
 (segment (start 36.195 33.02) (end 36.902106 33.02) (width 0.25) (layer F.Cu) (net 8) (status 10))
 (segment (start 41.91 34.29) (end 36.195 34.29) (width 0.25) (layer F.Cu) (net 9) (status 20))
 (segment (start 43.18 35.56) (end 41.91 34.29) (width 0.25) (layer F.Cu) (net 9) (status 10))
 (segment (start 38.735 38.1) (end 36.195 35.56) (width 0.25) (layer F.Cu) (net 10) (status 20))
 (segment (start 43.18 38.1) (end 38.735 38.1) (width 0.25) (layer F.Cu) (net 10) (status 10))
 (segment (start 92.71 36.31) (end 92.71 35.56) (width 0.25) (layer F.Cu) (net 11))
 (segment (start 94.520885 38.120885) (end 92.71 36.31) (width 0.25) (layer F.Cu) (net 11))
 (segment (start 99.552017 38.120885) (end 94.520885 38.120885) (width 0.25) (layer F.Cu) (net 11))
 (segment (start 98.917018 34.945884) (end 99.552019 35.580885) (width 0.25) (layer F.Cu) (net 12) (status 30))
 (segment (start 98.261132 34.29) (end 92.71 34.29) (width 0.25) (layer F.Cu) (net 12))
 (segment (start 99.552017 35.580885) (end 98.261132 34.29) (width 0.25) (layer F.Cu) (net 12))
 (segment (start 99.552018 33.040885) (end 98.917018 33.675885) (width 0.25) (layer F.Cu) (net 13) (status 30))
 (segment (start 99.531132 33.02) (end 99.552017 33.040885) (width 0.25) (layer F.Cu) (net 13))
 (segment (start 92.71 33.02) (end 99.531132 33.02) (width 0.25) (layer F.Cu) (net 13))
 (segment (start 98.349936 30.500884) (end 97.079937 31.770885) (width 0.25) (layer F.Cu) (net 14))
 (segment (start 99.552017 30.500884) (end 98.349936 30.500884) (width 0.25) (layer F.Cu) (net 14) (status 10))
 (segment (start 97.059052 31.75) (end 92.71 31.75) (width 0.25) (layer F.Cu) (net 14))
 (segment (start 97.079937 31.770885) (end 97.059052 31.75) (width 0.25) (layer F.Cu) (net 14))
 (segment (start 95.229115 27.960885) (end 92.71 30.48) (width 0.25) (layer F.Cu) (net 15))
 (segment (start 99.552017 27.960885) (end 95.229115 27.960885) (width 0.25) (layer F.Cu) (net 15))
 (segment (start 88.693517 38.120885) (end 91.233518 35.580884) (width 0.25) (layer F.Cu) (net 16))
 (segment (start 84.312018 38.120885) (end 88.693517 38.120885) (width 0.25) (layer F.Cu) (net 16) (status 10))
 (segment (start 84.312018 35.580885) (end 84.947018 34.945885) (width 0.25) (layer F.Cu) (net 17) (status 30))
 (segment (start 89.963518 35.580885) (end 91.233518 34.310885) (width 0.25) (layer F.Cu) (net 17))
 (segment (start 84.312018 35.580885) (end 89.963518 35.580885) (width 0.25) (layer F.Cu) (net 17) (status 10))
 (segment (start 84.312017 33.040885) (end 91.233518 33.040885) (width 0.25) (layer F.Cu) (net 18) (status 10))
 (segment (start 85.582018 31.770884) (end 91.233518 31.770884) (width 0.25) (layer F.Cu) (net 19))
 (segment (start 84.312018 30.500884) (end 85.582018 31.770884) (width 0.25) (layer F.Cu) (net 19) (status 10))
 (segment (start 89.646018 30.500885) (end 91.233518 30.500885) (width 0.25) (layer F.Cu) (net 20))
 (segment (start 84.312018 27.960885) (end 87.106017 27.960885) (width 0.25) (layer F.Cu) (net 20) (status 10))
 (segment (start 87.106017 27.960885) (end 89.646018 30.500885) (width 0.25) (layer F.Cu) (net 20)))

